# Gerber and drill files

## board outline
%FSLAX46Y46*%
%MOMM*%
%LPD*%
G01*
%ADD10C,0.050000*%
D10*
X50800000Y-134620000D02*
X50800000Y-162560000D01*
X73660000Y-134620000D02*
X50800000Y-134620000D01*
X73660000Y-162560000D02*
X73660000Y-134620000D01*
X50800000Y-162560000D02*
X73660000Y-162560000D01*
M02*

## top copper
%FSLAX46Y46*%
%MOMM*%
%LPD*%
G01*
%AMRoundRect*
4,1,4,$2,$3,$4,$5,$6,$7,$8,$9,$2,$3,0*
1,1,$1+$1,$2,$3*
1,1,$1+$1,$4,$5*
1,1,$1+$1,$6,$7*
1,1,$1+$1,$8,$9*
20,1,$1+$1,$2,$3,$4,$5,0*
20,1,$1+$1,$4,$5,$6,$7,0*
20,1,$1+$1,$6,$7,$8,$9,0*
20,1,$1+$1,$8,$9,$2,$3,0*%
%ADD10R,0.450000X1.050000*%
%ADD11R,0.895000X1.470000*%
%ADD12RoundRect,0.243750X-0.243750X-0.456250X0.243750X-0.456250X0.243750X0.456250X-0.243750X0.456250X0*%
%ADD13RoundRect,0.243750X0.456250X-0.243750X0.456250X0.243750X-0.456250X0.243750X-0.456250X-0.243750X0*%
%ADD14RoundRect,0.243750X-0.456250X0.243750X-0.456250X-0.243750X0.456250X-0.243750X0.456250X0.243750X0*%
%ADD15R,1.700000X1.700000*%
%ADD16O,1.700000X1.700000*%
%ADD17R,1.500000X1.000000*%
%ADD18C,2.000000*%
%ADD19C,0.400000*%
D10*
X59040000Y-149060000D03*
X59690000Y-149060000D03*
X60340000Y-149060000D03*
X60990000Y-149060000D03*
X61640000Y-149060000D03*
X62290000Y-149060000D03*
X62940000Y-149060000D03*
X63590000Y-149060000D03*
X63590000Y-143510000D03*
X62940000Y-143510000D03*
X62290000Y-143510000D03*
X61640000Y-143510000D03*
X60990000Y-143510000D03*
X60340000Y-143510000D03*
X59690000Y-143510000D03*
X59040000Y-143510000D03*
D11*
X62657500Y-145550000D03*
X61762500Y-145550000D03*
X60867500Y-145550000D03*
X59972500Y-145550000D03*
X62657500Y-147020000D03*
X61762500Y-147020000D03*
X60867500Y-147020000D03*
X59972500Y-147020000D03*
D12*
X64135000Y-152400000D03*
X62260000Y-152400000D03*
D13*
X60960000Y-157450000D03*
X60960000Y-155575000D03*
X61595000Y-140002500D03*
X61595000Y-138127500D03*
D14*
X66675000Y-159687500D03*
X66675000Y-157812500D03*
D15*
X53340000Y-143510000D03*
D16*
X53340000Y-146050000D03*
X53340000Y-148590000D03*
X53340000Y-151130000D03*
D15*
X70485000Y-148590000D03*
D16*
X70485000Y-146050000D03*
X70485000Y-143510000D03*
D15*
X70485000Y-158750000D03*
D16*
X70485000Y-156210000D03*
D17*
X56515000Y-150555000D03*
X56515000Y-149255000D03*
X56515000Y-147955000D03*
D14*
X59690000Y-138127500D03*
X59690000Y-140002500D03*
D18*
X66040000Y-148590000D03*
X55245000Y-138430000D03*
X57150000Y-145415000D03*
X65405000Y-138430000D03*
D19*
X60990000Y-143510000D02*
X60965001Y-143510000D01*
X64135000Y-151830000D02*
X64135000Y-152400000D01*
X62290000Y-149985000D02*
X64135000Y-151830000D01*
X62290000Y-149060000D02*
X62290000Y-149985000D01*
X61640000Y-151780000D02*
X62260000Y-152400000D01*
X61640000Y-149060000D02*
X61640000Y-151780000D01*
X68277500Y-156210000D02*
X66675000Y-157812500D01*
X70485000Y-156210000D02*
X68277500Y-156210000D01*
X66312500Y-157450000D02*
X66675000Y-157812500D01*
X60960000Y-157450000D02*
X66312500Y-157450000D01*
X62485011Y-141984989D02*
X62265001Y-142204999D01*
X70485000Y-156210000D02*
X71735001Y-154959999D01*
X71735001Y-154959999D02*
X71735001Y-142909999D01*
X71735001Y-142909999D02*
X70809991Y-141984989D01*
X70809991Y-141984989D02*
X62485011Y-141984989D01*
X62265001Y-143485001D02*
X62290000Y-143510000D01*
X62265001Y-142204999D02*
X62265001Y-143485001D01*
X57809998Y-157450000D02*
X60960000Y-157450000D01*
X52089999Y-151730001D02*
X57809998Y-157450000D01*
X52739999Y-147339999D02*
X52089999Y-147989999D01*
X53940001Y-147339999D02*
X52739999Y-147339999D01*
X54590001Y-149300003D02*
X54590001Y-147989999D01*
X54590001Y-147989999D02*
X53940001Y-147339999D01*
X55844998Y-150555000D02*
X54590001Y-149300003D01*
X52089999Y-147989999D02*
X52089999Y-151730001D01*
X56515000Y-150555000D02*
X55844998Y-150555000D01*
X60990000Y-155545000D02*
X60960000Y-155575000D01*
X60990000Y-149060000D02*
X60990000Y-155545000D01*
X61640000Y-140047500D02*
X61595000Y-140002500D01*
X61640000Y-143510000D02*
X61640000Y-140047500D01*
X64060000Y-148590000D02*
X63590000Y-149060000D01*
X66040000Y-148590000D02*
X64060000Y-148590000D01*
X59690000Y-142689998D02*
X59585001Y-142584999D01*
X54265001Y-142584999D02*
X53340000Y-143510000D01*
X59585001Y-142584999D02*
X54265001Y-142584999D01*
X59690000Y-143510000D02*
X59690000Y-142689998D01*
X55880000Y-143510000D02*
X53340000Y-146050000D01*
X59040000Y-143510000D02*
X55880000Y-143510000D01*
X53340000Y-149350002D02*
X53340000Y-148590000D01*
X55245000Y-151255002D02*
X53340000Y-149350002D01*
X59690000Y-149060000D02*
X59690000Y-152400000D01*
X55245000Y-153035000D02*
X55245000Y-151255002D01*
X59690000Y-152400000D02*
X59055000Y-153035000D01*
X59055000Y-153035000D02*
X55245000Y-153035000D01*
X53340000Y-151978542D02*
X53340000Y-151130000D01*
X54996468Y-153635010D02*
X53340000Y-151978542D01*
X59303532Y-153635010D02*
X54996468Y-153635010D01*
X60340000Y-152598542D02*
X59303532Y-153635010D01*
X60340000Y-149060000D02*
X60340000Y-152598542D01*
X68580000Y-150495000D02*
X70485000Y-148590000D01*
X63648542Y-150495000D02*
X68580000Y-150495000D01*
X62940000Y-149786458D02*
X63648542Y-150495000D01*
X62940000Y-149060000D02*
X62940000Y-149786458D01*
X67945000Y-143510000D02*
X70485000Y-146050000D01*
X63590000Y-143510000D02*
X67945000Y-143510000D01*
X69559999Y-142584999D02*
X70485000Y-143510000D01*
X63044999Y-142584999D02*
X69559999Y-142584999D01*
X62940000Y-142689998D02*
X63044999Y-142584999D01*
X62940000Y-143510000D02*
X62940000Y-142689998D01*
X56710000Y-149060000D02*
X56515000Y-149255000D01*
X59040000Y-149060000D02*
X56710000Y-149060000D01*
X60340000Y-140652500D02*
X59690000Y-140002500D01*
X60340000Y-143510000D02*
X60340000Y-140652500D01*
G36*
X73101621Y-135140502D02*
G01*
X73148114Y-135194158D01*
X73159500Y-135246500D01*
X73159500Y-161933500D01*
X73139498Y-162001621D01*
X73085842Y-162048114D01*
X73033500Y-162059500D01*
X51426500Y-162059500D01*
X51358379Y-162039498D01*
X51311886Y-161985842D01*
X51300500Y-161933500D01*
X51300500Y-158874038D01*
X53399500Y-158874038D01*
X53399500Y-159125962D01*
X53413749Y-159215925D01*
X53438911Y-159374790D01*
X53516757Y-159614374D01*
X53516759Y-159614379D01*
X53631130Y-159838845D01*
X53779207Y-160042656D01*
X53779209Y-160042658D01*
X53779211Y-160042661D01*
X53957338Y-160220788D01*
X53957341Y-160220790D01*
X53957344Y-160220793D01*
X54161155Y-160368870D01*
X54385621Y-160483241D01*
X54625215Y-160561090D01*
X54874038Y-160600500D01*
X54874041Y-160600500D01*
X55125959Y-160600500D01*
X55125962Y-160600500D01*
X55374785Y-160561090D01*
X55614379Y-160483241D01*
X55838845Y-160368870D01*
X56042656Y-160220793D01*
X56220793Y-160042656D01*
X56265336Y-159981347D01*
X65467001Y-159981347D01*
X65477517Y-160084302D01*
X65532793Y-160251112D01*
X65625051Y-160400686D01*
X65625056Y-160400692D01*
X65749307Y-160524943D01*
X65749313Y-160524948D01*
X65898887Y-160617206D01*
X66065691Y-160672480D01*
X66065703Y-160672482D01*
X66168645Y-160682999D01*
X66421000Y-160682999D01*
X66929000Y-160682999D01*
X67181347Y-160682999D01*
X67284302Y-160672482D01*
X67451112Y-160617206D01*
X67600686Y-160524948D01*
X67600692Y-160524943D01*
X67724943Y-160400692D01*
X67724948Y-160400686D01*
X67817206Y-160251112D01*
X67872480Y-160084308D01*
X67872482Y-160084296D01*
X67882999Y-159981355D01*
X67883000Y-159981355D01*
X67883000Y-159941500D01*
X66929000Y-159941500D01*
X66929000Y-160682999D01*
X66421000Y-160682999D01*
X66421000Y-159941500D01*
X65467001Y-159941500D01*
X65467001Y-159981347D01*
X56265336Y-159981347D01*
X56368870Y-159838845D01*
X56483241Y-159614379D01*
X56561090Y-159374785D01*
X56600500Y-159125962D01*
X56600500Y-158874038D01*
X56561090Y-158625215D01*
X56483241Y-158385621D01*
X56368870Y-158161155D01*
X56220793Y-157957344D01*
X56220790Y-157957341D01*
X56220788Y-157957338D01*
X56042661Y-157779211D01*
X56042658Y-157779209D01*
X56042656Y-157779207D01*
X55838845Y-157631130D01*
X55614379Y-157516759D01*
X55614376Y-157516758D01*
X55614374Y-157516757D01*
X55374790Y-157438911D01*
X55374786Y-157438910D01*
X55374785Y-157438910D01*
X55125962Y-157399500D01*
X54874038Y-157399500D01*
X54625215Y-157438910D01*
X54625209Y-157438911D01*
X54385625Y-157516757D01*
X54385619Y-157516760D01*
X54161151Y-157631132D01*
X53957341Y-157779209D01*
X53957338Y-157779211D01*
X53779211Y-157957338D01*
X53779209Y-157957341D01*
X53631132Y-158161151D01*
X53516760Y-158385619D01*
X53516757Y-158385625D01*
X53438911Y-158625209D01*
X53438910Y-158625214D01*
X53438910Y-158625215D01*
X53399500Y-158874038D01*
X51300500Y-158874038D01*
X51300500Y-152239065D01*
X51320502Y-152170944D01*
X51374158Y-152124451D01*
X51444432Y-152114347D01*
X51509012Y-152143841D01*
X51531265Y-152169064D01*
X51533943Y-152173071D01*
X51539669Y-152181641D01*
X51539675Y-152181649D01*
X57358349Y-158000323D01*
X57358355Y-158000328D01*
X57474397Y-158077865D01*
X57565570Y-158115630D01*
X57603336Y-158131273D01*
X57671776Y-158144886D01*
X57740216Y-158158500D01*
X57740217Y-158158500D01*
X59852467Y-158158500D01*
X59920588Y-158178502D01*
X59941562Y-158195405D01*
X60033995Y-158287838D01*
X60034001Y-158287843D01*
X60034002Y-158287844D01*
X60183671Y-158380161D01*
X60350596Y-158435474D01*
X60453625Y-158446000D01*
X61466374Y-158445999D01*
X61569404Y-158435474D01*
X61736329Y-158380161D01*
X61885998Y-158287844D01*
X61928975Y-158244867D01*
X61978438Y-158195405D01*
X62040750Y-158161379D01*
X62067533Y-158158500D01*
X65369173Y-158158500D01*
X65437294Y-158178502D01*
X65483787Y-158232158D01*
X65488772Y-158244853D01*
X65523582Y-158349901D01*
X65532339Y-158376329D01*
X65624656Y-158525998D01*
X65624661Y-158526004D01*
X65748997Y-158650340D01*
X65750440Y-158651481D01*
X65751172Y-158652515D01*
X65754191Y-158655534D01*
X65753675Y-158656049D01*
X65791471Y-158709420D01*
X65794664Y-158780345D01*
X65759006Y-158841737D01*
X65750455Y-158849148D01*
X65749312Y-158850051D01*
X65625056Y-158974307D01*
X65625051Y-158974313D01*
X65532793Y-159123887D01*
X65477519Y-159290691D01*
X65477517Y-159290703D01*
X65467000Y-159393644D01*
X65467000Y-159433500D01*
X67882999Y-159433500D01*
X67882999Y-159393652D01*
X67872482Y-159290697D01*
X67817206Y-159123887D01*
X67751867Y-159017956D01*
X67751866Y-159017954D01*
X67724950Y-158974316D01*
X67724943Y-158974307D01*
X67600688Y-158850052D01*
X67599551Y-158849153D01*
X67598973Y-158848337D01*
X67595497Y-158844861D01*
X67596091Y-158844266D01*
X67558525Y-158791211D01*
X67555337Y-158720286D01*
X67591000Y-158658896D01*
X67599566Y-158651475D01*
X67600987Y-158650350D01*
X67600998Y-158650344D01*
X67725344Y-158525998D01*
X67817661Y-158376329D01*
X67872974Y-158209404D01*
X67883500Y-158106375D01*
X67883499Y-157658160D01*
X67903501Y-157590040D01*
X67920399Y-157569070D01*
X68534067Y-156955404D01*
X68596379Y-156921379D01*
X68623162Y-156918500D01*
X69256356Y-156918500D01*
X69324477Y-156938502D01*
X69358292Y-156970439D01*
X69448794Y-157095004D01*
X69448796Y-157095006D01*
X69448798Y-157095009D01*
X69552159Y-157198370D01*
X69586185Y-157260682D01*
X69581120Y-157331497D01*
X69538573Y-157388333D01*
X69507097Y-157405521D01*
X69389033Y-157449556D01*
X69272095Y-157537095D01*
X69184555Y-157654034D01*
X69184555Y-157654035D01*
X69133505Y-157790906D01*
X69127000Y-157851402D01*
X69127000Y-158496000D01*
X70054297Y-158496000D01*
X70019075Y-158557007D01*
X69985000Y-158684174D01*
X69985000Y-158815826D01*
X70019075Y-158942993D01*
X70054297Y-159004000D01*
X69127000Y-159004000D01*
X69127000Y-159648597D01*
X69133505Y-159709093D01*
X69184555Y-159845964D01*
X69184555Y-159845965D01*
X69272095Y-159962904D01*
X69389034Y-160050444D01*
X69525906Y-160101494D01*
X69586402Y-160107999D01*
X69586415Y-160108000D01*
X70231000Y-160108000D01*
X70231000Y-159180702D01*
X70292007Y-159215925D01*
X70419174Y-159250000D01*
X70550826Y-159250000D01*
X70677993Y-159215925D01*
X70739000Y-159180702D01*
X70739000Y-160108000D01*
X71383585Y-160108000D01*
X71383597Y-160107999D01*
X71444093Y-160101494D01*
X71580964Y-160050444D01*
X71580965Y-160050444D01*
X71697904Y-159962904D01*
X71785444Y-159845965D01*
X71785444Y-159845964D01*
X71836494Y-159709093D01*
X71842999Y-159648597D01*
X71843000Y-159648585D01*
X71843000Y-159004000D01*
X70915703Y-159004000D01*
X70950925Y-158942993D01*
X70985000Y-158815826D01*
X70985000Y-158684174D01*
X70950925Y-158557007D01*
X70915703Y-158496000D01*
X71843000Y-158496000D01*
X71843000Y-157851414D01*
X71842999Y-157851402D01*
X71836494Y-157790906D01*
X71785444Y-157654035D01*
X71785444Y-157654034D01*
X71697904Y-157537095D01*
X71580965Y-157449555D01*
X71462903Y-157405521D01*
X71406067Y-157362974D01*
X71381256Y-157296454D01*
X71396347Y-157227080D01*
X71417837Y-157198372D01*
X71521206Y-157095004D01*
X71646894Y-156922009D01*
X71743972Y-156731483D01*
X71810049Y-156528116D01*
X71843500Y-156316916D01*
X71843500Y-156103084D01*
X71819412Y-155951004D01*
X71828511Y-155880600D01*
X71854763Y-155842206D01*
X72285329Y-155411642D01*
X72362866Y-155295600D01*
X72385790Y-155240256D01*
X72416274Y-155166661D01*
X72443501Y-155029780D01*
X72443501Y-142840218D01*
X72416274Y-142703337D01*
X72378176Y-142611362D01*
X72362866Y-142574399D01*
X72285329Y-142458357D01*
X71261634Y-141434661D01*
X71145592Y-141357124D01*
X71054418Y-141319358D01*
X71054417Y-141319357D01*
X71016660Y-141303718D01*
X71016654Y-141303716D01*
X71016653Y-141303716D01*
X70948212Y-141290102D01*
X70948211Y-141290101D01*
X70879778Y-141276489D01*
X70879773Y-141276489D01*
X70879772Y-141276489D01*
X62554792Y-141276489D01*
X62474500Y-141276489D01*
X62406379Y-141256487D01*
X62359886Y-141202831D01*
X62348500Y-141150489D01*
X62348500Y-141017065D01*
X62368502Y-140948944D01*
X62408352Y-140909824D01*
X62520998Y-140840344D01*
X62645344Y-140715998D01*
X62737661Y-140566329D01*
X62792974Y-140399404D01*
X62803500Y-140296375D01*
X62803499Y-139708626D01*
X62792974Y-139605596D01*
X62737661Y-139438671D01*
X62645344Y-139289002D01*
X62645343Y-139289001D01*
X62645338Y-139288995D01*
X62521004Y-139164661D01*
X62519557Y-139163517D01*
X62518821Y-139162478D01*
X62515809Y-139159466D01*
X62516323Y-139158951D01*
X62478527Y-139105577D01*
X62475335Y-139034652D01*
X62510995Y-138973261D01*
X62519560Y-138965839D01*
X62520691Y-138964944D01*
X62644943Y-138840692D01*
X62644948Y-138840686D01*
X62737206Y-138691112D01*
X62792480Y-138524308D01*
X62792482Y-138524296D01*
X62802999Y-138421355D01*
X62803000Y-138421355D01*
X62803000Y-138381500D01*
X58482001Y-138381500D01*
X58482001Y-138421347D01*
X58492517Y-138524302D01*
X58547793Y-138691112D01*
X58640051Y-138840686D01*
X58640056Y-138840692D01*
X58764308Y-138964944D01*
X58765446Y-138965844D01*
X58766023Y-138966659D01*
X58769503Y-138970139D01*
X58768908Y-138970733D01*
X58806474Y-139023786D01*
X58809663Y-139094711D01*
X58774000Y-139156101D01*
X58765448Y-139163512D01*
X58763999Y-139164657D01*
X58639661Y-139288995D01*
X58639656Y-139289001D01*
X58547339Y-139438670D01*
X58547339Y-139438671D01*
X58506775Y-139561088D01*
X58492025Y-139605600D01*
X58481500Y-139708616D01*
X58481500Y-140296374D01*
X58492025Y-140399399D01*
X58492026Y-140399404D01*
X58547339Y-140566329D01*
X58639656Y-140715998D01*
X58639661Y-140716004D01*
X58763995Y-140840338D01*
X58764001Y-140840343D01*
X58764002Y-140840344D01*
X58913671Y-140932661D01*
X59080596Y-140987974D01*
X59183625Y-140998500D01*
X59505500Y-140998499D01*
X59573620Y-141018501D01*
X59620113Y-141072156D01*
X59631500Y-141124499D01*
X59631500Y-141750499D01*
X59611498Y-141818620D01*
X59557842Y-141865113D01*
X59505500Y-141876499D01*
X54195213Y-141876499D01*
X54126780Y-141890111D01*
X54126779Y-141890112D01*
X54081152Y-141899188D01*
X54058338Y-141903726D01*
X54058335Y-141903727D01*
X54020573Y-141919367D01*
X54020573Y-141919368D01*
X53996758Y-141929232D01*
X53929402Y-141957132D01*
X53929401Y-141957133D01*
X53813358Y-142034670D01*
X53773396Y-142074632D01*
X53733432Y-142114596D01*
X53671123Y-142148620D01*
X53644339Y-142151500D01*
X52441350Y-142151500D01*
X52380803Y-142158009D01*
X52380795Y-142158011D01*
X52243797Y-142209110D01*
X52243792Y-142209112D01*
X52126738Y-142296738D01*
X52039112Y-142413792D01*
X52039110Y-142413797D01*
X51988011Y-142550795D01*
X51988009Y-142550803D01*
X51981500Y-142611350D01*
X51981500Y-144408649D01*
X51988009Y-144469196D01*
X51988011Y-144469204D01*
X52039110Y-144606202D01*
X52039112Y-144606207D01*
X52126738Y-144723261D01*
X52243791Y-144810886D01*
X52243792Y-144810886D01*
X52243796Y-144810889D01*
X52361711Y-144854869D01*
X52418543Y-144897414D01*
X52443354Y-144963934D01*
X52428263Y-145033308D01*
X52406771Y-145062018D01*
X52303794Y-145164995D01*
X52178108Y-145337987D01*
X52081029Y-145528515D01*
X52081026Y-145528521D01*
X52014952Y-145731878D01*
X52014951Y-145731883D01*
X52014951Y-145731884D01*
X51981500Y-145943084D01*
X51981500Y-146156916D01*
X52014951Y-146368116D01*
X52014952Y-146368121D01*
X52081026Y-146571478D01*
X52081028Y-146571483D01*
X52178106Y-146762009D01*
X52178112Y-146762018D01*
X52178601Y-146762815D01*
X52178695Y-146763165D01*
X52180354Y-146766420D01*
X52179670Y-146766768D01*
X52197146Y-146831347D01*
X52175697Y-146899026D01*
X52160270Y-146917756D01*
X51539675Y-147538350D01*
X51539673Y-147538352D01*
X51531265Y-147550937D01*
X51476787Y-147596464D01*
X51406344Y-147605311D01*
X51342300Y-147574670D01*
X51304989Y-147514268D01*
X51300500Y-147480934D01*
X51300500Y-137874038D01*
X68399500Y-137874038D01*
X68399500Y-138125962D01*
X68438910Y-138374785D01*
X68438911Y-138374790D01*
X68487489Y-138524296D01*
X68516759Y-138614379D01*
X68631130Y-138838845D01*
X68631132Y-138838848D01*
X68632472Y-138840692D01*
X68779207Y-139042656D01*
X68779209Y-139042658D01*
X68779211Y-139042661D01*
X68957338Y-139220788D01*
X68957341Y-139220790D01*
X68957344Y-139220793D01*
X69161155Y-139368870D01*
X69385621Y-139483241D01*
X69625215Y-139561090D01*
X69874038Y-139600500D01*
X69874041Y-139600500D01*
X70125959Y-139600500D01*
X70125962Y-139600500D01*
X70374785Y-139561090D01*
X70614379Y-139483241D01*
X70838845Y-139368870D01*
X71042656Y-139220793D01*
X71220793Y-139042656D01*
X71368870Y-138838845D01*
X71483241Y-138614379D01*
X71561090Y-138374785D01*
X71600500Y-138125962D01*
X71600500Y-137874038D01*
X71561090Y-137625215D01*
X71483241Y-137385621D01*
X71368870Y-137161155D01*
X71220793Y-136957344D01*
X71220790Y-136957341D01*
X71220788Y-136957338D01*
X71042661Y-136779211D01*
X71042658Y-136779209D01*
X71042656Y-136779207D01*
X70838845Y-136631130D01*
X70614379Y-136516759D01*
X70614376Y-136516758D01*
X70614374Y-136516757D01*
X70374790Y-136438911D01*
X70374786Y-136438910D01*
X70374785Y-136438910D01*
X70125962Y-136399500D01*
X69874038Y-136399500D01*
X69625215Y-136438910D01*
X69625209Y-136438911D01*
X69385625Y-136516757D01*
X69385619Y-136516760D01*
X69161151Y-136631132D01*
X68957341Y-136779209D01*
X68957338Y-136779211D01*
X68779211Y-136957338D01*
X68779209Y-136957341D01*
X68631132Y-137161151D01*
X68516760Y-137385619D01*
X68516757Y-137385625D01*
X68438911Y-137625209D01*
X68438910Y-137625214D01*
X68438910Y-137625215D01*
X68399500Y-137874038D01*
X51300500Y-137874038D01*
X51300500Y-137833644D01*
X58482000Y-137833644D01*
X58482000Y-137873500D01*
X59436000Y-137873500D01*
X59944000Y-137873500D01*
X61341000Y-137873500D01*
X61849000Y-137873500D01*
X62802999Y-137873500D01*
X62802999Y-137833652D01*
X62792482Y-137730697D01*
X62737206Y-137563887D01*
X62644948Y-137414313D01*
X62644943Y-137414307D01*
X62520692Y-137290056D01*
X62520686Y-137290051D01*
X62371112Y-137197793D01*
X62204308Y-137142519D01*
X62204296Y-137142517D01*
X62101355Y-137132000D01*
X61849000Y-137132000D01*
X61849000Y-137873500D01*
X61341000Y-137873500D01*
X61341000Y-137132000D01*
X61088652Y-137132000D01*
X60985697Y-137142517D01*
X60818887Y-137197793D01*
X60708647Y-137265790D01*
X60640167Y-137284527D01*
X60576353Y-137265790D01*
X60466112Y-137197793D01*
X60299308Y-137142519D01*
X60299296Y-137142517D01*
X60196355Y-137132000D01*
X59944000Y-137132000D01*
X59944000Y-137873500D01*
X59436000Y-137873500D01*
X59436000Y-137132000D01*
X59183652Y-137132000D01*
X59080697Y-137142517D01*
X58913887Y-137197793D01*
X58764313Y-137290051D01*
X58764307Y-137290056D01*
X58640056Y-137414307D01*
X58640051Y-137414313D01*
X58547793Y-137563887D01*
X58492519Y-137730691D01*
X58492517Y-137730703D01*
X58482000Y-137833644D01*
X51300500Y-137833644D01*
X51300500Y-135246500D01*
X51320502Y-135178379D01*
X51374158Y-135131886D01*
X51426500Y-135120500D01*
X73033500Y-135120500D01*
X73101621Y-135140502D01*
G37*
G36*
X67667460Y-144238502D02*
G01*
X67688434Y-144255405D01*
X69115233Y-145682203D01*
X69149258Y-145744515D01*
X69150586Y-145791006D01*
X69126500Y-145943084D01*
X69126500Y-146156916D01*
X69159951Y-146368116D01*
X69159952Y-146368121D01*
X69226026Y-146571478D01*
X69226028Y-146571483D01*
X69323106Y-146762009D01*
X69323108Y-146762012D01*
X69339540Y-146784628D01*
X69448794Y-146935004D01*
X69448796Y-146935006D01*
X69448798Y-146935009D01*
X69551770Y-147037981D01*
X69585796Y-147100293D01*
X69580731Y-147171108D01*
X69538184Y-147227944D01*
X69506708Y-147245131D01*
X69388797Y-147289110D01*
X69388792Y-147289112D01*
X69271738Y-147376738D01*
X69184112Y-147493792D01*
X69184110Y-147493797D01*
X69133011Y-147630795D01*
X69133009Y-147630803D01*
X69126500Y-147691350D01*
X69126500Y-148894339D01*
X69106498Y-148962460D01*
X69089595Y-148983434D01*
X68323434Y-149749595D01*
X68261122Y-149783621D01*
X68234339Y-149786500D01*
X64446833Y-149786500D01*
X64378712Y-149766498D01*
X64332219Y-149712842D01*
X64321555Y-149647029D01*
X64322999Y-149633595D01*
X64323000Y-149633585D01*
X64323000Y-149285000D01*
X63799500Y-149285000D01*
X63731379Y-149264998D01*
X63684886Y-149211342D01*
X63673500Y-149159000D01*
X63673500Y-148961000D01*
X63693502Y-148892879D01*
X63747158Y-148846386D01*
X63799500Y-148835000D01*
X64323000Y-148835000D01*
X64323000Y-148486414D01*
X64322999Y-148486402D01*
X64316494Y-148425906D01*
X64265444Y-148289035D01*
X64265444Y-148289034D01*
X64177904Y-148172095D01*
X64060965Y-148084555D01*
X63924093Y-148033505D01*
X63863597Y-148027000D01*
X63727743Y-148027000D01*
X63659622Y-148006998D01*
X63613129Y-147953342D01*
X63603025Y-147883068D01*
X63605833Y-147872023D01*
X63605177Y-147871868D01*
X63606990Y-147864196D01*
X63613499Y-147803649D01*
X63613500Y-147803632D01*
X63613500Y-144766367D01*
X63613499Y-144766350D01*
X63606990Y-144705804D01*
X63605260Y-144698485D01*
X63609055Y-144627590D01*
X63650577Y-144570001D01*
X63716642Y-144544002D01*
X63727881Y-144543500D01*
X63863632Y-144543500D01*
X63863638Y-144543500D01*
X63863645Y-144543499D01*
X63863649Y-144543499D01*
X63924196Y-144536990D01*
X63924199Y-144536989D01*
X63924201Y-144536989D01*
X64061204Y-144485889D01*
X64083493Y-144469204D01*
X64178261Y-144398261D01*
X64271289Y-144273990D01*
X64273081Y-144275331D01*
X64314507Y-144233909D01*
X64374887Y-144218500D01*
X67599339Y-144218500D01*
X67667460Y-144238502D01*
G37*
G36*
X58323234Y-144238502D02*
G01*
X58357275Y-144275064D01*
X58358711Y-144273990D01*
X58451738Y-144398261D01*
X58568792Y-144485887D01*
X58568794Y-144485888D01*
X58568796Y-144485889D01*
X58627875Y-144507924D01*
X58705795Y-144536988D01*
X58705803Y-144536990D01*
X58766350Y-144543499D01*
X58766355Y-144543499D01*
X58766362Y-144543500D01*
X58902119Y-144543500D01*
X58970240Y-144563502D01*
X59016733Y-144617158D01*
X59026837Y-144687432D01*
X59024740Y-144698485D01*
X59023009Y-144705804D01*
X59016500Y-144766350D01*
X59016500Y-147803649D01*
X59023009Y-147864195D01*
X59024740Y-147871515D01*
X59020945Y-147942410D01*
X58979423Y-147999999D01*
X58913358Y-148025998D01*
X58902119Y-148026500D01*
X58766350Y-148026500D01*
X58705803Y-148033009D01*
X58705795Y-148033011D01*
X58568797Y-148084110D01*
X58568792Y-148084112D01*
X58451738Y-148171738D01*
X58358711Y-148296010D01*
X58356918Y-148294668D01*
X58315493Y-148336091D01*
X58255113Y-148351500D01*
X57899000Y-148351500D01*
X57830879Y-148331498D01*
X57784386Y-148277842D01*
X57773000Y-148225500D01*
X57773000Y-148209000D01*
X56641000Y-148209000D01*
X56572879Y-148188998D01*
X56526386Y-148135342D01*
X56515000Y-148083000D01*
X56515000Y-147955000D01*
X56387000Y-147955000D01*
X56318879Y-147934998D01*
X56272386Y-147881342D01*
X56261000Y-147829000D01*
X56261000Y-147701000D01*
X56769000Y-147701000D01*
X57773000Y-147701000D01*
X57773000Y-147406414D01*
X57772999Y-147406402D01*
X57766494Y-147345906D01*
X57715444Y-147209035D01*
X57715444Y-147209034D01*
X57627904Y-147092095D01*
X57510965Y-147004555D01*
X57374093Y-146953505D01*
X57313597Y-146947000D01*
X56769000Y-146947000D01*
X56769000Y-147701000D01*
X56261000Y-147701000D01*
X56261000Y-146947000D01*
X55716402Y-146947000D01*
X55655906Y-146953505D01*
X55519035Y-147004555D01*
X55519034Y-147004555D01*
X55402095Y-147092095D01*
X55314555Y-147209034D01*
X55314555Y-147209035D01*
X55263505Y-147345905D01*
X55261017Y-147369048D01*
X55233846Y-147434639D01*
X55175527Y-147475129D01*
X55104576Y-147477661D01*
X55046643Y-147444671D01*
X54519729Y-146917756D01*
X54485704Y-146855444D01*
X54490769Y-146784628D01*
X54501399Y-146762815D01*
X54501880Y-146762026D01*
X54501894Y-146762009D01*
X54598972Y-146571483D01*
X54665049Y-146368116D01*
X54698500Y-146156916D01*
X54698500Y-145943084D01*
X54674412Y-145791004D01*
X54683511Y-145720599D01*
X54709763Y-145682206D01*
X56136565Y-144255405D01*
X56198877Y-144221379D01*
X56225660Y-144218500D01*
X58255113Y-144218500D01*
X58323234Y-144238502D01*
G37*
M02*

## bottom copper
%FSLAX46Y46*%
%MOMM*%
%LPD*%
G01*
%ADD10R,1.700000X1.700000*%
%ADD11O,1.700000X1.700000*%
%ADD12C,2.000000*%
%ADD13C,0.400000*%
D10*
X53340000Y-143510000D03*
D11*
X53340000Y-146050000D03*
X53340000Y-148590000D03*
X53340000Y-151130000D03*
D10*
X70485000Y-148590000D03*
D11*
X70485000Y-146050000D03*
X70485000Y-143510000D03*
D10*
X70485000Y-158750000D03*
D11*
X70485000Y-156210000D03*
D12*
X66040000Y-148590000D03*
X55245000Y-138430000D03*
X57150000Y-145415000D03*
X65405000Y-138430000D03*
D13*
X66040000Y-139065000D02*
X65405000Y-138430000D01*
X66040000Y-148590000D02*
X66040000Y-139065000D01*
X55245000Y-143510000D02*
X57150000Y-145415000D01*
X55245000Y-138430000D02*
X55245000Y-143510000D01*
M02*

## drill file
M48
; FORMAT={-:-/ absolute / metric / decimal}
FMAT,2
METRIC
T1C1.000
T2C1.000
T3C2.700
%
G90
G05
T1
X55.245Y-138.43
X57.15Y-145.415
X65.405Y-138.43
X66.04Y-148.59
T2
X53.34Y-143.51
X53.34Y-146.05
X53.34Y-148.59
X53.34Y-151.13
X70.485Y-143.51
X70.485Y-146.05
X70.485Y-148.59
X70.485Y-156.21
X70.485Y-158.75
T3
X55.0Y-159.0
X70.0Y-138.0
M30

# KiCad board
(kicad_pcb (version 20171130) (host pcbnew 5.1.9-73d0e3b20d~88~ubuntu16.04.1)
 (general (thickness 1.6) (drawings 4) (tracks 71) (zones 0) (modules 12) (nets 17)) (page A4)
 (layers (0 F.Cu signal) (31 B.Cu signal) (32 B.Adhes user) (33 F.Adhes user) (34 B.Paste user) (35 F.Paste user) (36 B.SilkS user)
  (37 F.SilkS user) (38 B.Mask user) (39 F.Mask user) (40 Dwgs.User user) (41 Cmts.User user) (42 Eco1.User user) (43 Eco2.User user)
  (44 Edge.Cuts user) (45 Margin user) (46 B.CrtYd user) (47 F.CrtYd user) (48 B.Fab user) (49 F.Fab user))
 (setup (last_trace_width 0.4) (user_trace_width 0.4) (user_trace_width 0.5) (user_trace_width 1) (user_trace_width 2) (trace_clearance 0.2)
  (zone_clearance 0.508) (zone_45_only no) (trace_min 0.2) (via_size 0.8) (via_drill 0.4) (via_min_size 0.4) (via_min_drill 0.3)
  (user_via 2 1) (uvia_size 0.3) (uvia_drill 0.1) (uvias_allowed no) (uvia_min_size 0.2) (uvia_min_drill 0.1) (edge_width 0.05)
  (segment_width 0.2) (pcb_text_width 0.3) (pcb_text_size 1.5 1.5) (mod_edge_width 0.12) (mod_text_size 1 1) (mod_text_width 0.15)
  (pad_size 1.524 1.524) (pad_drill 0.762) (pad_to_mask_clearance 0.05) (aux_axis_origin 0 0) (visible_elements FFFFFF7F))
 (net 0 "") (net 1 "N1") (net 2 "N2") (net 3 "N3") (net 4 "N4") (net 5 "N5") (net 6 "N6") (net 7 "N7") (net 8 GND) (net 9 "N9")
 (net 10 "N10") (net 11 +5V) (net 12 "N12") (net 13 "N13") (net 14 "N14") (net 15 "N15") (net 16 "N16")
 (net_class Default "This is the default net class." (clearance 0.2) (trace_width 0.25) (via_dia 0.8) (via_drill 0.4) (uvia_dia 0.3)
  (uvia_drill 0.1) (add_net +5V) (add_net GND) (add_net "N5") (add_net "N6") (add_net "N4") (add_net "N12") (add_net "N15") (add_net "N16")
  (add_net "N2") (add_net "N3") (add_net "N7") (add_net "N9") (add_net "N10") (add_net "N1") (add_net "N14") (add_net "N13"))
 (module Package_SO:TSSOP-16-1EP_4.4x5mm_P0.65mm (layer F.Cu) (at 61.315 146.285 90)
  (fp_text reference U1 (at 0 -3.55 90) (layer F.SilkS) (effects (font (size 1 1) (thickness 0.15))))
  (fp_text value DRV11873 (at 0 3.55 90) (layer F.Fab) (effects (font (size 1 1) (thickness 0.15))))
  (pad 1 smd rect (at -2.775 -2.275 90) (size 1.05 0.45) (layers F.Cu F.Paste F.Mask) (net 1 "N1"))
  (pad 2 smd rect (at -2.775 -1.625 90) (size 1.05 0.45) (layers F.Cu F.Paste F.Mask) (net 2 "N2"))
  (pad 3 smd rect (at -2.775 -0.975 90) (size 1.05 0.45) (layers F.Cu F.Paste F.Mask) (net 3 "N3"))
  (pad 4 smd rect (at -2.775 -0.325 90) (size 1.05 0.45) (layers F.Cu F.Paste F.Mask) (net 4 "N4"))
  (pad 5 smd rect (at -2.775 0.325 90) (size 1.05 0.45) (layers F.Cu F.Paste F.Mask) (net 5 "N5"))
  (pad 6 smd rect (at -2.775 0.975 90) (size 1.05 0.45) (layers F.Cu F.Paste F.Mask) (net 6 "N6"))
  (pad 7 smd rect (at -2.775 1.625 90) (size 1.05 0.45) (layers F.Cu F.Paste F.Mask) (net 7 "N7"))
  (pad 8 smd rect (at -2.775 2.275 90) (size 1.05 0.45) (layers F.Cu F.Paste F.Mask) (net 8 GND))
  (pad 9 smd rect (at 2.775 2.275 90) (size 1.05 0.45) (layers F.Cu F.Paste F.Mask) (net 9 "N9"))
  (pad 10 smd rect (at 2.775 1.625 90) (size 1.05 0.45) (layers F.Cu F.Paste F.Mask) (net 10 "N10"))
  (pad 11 smd rect (at 2.775 0.975 90) (size 1.05 0.45) (layers F.Cu F.Paste F.Mask) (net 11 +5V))
  (pad 12 smd rect (at 2.775 0.325 90) (size 1.05 0.45) (layers F.Cu F.Paste F.Mask) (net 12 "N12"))
  (pad 13 smd rect (at 2.775 -0.325 90) (size 1.05 0.45) (layers F.Cu F.Paste F.Mask) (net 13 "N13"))
  (pad 14 smd rect (at 2.775 -0.975 90) (size 1.05 0.45) (layers F.Cu F.Paste F.Mask) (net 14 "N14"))
  (pad 15 smd rect (at 2.775 -1.625 90) (size 1.05 0.45) (layers F.Cu F.Paste F.Mask) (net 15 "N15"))
  (pad 16 smd rect (at 2.775 -2.275 90) (size 1.05 0.45) (layers F.Cu F.Paste F.Mask) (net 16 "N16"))
  (pad 17 smd rect (at 0.735 1.3425 90) (size 1.47 0.895) (layers F.Cu F.Paste F.Mask) (solder_paste_margin_ratio -0.2))
  (pad 17 smd rect (at 0.735 0.4475 90) (size 1.47 0.895) (layers F.Cu F.Paste F.Mask) (solder_paste_margin_ratio -0.2))
  (pad 17 smd rect (at 0.735 -0.4475 90) (size 1.47 0.895) (layers F.Cu F.Paste F.Mask) (solder_paste_margin_ratio -0.2))
  (pad 17 smd rect (at 0.735 -1.3425 90) (size 1.47 0.895) (layers F.Cu F.Paste F.Mask) (solder_paste_margin_ratio -0.2))
  (pad 17 smd rect (at -0.735 1.3425 90) (size 1.47 0.895) (layers F.Cu F.Paste F.Mask) (solder_paste_margin_ratio -0.2))
  (pad 17 smd rect (at -0.735 0.4475 90) (size 1.47 0.895) (layers F.Cu F.Paste F.Mask) (solder_paste_margin_ratio -0.2))
  (pad 17 smd rect (at -0.735 -0.4475 90) (size 1.47 0.895) (layers F.Cu F.Paste F.Mask) (solder_paste_margin_ratio -0.2))
  (pad 17 smd rect (at -0.735 -1.3425 90) (size 1.47 0.895) (layers F.Cu F.Paste F.Mask) (solder_paste_margin_ratio -0.2)))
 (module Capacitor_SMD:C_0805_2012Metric (layer F.Cu) (at 63.1975 152.4)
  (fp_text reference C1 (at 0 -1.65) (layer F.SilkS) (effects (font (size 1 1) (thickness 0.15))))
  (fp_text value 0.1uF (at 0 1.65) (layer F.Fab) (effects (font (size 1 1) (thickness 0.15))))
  (pad 2 smd roundrect (at 0.9375 0) (size 0.975 1.4) (layers F.Cu F.Paste F.Mask) (roundrect_rratio 0.25) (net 6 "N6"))
  (pad 1 smd roundrect (at -0.9375 0) (size 0.975 1.4) (layers F.Cu F.Paste F.Mask) (roundrect_rratio 0.25) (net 5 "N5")))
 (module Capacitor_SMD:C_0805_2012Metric (layer F.Cu) (at 60.96 156.5125 90)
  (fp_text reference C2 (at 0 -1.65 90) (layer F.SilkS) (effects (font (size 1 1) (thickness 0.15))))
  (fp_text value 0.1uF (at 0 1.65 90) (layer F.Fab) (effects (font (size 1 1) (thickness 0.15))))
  (pad 1 smd roundrect (at -0.9375 0 90) (size 0.975 1.4) (layers F.Cu F.Paste F.Mask) (roundrect_rratio 0.25) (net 11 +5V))
  (pad 2 smd roundrect (at 0.9375 0 90) (size 0.975 1.4) (layers F.Cu F.Paste F.Mask) (roundrect_rratio 0.25) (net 4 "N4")))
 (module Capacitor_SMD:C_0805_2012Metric (layer F.Cu) (at 61.595 139.065 90)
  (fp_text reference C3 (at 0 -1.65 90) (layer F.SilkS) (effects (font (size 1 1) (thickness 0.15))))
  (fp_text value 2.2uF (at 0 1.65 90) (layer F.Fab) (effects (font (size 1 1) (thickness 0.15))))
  (pad 1 smd roundrect (at -0.9375 0 90) (size 0.975 1.4) (layers F.Cu F.Paste F.Mask) (roundrect_rratio 0.25) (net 12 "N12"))
  (pad 2 smd roundrect (at 0.9375 0 90) (size 0.975 1.4) (layers F.Cu F.Paste F.Mask) (roundrect_rratio 0.25) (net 8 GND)))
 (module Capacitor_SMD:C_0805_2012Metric (layer F.Cu) (at 66.675 158.75 270)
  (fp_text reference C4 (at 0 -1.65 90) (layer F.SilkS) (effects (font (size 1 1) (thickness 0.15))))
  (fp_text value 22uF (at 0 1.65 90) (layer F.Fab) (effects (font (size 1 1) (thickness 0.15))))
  (pad 2 smd roundrect (at 0.9375 0 270) (size 0.975 1.4) (layers F.Cu F.Paste F.Mask) (roundrect_rratio 0.25) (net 8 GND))
  (pad 1 smd roundrect (at -0.9375 0 270) (size 0.975 1.4) (layers F.Cu F.Paste F.Mask) (roundrect_rratio 0.25) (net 11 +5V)))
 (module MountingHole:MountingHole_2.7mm (layer F.Cu) (at 70 138)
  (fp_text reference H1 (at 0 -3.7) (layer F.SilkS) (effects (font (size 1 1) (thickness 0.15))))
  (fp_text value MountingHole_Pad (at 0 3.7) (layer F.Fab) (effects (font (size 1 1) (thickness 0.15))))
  (pad 1 np_thru_hole circle (at 0 0) (size 2.7 2.7) (drill 2.7) (layers *.Cu *.Mask) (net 8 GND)))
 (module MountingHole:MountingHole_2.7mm (layer F.Cu) (at 55 159)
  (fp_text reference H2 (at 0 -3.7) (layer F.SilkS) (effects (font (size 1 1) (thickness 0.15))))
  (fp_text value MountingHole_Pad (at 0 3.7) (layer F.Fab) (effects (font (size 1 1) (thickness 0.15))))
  (pad 1 np_thru_hole circle (at 0 0) (size 2.7 2.7) (drill 2.7) (layers *.Cu *.Mask) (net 8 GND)))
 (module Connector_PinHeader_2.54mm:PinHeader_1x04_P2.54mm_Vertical (layer F.Cu) (at 53.34 143.51)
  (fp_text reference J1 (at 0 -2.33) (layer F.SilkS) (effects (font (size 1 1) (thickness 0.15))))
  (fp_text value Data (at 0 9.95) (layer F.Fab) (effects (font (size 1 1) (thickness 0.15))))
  (pad 1 thru_hole rect (at 0 0) (size 1.7 1.7) (drill 1) (layers *.Cu *.Mask) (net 15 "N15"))
  (pad 2 thru_hole oval (at 0 2.54) (size 1.7 1.7) (drill 1) (layers *.Cu *.Mask) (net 16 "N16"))
  (pad 3 thru_hole oval (at 0 5.08) (size 1.7 1.7) (drill 1) (layers *.Cu *.Mask) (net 2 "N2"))
  (pad 4 thru_hole oval (at 0 7.62) (size 1.7 1.7) (drill 1) (layers *.Cu *.Mask) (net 3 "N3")))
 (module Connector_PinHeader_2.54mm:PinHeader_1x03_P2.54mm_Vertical (layer F.Cu) (at 70.485 148.59 180)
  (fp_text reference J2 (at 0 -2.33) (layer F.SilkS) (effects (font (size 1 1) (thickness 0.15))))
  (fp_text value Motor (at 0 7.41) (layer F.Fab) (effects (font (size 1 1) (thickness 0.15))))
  (pad 1 thru_hole rect (at 0 0 180) (size 1.7 1.7) (drill 1) (layers *.Cu *.Mask) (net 7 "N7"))
  (pad 2 thru_hole oval (at 0 2.54 180) (size 1.7 1.7) (drill 1) (layers *.Cu *.Mask) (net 9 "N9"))
  (pad 3 thru_hole oval (at 0 5.08 180) (size 1.7 1.7) (drill 1) (layers *.Cu *.Mask) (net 10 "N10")))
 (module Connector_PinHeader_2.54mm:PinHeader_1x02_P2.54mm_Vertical (layer F.Cu) (at 70.485 158.75 180)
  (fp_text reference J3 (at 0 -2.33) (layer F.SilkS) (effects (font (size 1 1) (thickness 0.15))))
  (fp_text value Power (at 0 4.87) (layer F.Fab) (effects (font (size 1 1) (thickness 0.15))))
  (pad 1 thru_hole rect (at 0 0 180) (size 1.7 1.7) (drill 1) (layers *.Cu *.Mask) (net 8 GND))
  (pad 2 thru_hole oval (at 0 2.54 180) (size 1.7 1.7) (drill 1) (layers *.Cu *.Mask) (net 11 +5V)))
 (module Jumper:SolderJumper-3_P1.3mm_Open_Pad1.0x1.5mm (layer F.Cu) (at 56.515 149.255 270)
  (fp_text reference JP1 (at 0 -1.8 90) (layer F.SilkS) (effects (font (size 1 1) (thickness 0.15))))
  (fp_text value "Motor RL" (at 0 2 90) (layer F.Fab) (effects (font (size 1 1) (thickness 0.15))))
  (pad 3 smd rect (at 1.3 0 270) (size 1 1.5) (layers F.Cu F.Mask) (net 11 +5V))
  (pad 2 smd rect (at 0 0 270) (size 1 1.5) (layers F.Cu F.Mask) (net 1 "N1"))
  (pad 1 smd rect (at -1.3 0 270) (size 1 1.5) (layers F.Cu F.Mask) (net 8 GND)))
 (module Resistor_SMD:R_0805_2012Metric (layer F.Cu) (at 59.69 139.065 270)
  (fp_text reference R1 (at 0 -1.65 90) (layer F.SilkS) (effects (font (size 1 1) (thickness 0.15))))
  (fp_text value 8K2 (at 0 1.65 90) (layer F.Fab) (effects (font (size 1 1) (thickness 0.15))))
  (pad 1 smd roundrect (at -0.9375 0 270) (size 0.975 1.4) (layers F.Cu F.Paste F.Mask) (roundrect_rratio 0.25) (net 8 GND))
  (pad 2 smd roundrect (at 0.9375 0 270) (size 0.975 1.4) (layers F.Cu F.Paste F.Mask) (roundrect_rratio 0.25) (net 14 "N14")))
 (gr_line (start 50.8 134.62) (end 50.8 162.56) (layer Edge.Cuts) (width 0.05))
 (gr_line (start 73.66 134.62) (end 50.8 134.62) (layer Edge.Cuts) (width 0.05))
 (gr_line (start 73.66 162.56) (end 73.66 134.62) (layer Edge.Cuts) (width 0.05))
 (gr_line (start 50.8 162.56) (end 73.66 162.56) (layer Edge.Cuts) (width 0.05))
 (via (at 66.04 148.59) (size 2) (drill 1) (layers F.Cu B.Cu) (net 8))
 (segment (start 60.99 143.51) (end 60.965001 143.51) (width 0.4) (layer F.Cu) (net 13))
 (segment (start 64.135 151.83) (end 64.135 152.4) (width 0.4) (layer F.Cu) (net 6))
 (segment (start 62.29 149.985) (end 64.135 151.83) (width 0.4) (layer F.Cu) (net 6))
 (segment (start 62.29 149.06) (end 62.29 149.985) (width 0.4) (layer F.Cu) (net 6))
 (segment (start 61.64 151.78) (end 62.26 152.4) (width 0.4) (layer F.Cu) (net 5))
 (segment (start 61.64 149.06) (end 61.64 151.78) (width 0.4) (layer F.Cu) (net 5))
 (segment (start 68.2775 156.21) (end 66.675 157.8125) (width 0.4) (layer F.Cu) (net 11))
 (segment (start 70.485 156.21) (end 68.2775 156.21) (width 0.4) (layer F.Cu) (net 11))
 (segment (start 66.3125 157.45) (end 66.675 157.8125) (width 0.4) (layer F.Cu) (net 11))
 (segment (start 60.96 157.45) (end 66.3125 157.45) (width 0.4) (layer F.Cu) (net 11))
 (segment (start 62.485011 141.984989) (end 62.265001 142.204999) (width 0.4) (layer F.Cu) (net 11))
 (segment (start 70.485 156.21) (end 71.735001 154.959999) (width 0.4) (layer F.Cu) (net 11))
 (segment (start 71.735001 154.959999) (end 71.735001 142.909999) (width 0.4) (layer F.Cu) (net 11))
 (segment (start 71.735001 142.909999) (end 70.809991 141.984989) (width 0.4) (layer F.Cu) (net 11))
 (segment (start 70.809991 141.984989) (end 62.485011 141.984989) (width 0.4) (layer F.Cu) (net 11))
 (segment (start 62.265001 143.485001) (end 62.29 143.51) (width 0.4) (layer F.Cu) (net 11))
 (segment (start 62.265001 142.204999) (end 62.265001 143.485001) (width 0.4) (layer F.Cu) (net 11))
 (segment (start 57.809998 157.45) (end 60.96 157.45) (width 0.4) (layer F.Cu) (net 11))
 (segment (start 52.089999 151.730001) (end 57.809998 157.45) (width 0.4) (layer F.Cu) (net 11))
 (segment (start 52.739999 147.339999) (end 52.089999 147.989999) (width 0.4) (layer F.Cu) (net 11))
 (segment (start 53.940001 147.339999) (end 52.739999 147.339999) (width 0.4) (layer F.Cu) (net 11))
 (segment (start 54.590001 149.300003) (end 54.590001 147.989999) (width 0.4) (layer F.Cu) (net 11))
 (segment (start 54.590001 147.989999) (end 53.940001 147.339999) (width 0.4) (layer F.Cu) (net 11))
 (segment (start 55.844998 150.555) (end 54.590001 149.300003) (width 0.4) (layer F.Cu) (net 11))
 (segment (start 52.089999 147.989999) (end 52.089999 151.730001) (width 0.4) (layer F.Cu) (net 11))
 (segment (start 56.515 150.555) (end 55.844998 150.555) (width 0.4) (layer F.Cu) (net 11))
 (segment (start 60.99 155.545) (end 60.96 155.575) (width 0.4) (layer F.Cu) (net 4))
 (segment (start 60.99 149.06) (end 60.99 155.545) (width 0.4) (layer F.Cu) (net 4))
 (segment (start 61.64 140.0475) (end 61.595 140.0025) (width 0.4) (layer F.Cu) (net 12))
 (segment (start 61.64 143.51) (end 61.64 140.0475) (width 0.4) (layer F.Cu) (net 12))
 (via (at 55.245 138.43) (size 2) (drill 1) (layers F.Cu B.Cu) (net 8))
 (via (at 57.15 145.415) (size 2) (drill 1) (layers F.Cu B.Cu) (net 8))
 (via (at 65.405 138.43) (size 2) (drill 1) (layers F.Cu B.Cu) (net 8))
 (segment (start 66.04 139.065) (end 65.405 138.43) (width 0.4) (layer B.Cu) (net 8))
 (segment (start 66.04 148.59) (end 66.04 139.065) (width 0.4) (layer B.Cu) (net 8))
 (segment (start 55.245 143.51) (end 57.15 145.415) (width 0.4) (layer B.Cu) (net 8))
 (segment (start 55.245 138.43) (end 55.245 143.51) (width 0.4) (layer B.Cu) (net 8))
 (segment (start 64.06 148.59) (end 63.59 149.06) (width 0.4) (layer F.Cu) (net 8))
 (segment (start 66.04 148.59) (end 64.06 148.59) (width 0.4) (layer F.Cu) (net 8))
 (segment (start 59.69 142.689998) (end 59.585001 142.584999) (width 0.4) (layer F.Cu) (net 15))
 (segment (start 54.265001 142.584999) (end 53.34 143.51) (width 0.4) (layer F.Cu) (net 15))
 (segment (start 59.585001 142.584999) (end 54.265001 142.584999) (width 0.4) (layer F.Cu) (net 15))
 (segment (start 59.69 143.51) (end 59.69 142.689998) (width 0.4) (layer F.Cu) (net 15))
 (segment (start 55.88 143.51) (end 53.34 146.05) (width 0.4) (layer F.Cu) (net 16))
 (segment (start 59.04 143.51) (end 55.88 143.51) (width 0.4) (layer F.Cu) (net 16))
 (segment (start 53.34 149.350002) (end 53.34 148.59) (width 0.4) (layer F.Cu) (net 2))
 (segment (start 55.245 151.255002) (end 53.34 149.350002) (width 0.4) (layer F.Cu) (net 2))
 (segment (start 59.69 149.06) (end 59.69 152.4) (width 0.4) (layer F.Cu) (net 2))
 (segment (start 55.245 153.035) (end 55.245 151.255002) (width 0.4) (layer F.Cu) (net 2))
 (segment (start 59.69 152.4) (end 59.055 153.035) (width 0.4) (layer F.Cu) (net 2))
 (segment (start 59.055 153.035) (end 55.245 153.035) (width 0.4) (layer F.Cu) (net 2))
 (segment (start 53.34 151.978542) (end 53.34 151.13) (width 0.4) (layer F.Cu) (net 3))
 (segment (start 54.996468 153.63501) (end 53.34 151.978542) (width 0.4) (layer F.Cu) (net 3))
 (segment (start 59.303532 153.63501) (end 54.996468 153.63501) (width 0.4) (layer F.Cu) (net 3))
 (segment (start 60.34 152.598542) (end 59.303532 153.63501) (width 0.4) (layer F.Cu) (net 3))
 (segment (start 60.34 149.06) (end 60.34 152.598542) (width 0.4) (layer F.Cu) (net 3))
 (segment (start 68.58 150.495) (end 70.485 148.59) (width 0.4) (layer F.Cu) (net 7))
 (segment (start 63.648542 150.495) (end 68.58 150.495) (width 0.4) (layer F.Cu) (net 7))
 (segment (start 62.94 149.786458) (end 63.648542 150.495) (width 0.4) (layer F.Cu) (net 7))
 (segment (start 62.94 149.06) (end 62.94 149.786458) (width 0.4) (layer F.Cu) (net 7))
 (segment (start 67.945 143.51) (end 70.485 146.05) (width 0.4) (layer F.Cu) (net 9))
 (segment (start 63.59 143.51) (end 67.945 143.51) (width 0.4) (layer F.Cu) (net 9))
 (segment (start 69.559999 142.584999) (end 70.485 143.51) (width 0.4) (layer F.Cu) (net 10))
 (segment (start 63.044999 142.584999) (end 69.559999 142.584999) (width 0.4) (layer F.Cu) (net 10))
 (segment (start 62.94 142.689998) (end 63.044999 142.584999) (width 0.4) (layer F.Cu) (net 10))
 (segment (start 62.94 143.51) (end 62.94 142.689998) (width 0.4) (layer F.Cu) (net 10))
 (segment (start 56.71 149.06) (end 56.515 149.255) (width 0.4) (layer F.Cu) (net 1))
 (segment (start 59.04 149.06) (end 56.71 149.06) (width 0.4) (layer F.Cu) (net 1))
 (segment (start 60.34 140.6525) (end 59.69 140.0025) (width 0.4) (layer F.Cu) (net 14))
 (segment (start 60.34 143.51) (end 60.34 140.6525) (width 0.4) (layer F.Cu) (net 14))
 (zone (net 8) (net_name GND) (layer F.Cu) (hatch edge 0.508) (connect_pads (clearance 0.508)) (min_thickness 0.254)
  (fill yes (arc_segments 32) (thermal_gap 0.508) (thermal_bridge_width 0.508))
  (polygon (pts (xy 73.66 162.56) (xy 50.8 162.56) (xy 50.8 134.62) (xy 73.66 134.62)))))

